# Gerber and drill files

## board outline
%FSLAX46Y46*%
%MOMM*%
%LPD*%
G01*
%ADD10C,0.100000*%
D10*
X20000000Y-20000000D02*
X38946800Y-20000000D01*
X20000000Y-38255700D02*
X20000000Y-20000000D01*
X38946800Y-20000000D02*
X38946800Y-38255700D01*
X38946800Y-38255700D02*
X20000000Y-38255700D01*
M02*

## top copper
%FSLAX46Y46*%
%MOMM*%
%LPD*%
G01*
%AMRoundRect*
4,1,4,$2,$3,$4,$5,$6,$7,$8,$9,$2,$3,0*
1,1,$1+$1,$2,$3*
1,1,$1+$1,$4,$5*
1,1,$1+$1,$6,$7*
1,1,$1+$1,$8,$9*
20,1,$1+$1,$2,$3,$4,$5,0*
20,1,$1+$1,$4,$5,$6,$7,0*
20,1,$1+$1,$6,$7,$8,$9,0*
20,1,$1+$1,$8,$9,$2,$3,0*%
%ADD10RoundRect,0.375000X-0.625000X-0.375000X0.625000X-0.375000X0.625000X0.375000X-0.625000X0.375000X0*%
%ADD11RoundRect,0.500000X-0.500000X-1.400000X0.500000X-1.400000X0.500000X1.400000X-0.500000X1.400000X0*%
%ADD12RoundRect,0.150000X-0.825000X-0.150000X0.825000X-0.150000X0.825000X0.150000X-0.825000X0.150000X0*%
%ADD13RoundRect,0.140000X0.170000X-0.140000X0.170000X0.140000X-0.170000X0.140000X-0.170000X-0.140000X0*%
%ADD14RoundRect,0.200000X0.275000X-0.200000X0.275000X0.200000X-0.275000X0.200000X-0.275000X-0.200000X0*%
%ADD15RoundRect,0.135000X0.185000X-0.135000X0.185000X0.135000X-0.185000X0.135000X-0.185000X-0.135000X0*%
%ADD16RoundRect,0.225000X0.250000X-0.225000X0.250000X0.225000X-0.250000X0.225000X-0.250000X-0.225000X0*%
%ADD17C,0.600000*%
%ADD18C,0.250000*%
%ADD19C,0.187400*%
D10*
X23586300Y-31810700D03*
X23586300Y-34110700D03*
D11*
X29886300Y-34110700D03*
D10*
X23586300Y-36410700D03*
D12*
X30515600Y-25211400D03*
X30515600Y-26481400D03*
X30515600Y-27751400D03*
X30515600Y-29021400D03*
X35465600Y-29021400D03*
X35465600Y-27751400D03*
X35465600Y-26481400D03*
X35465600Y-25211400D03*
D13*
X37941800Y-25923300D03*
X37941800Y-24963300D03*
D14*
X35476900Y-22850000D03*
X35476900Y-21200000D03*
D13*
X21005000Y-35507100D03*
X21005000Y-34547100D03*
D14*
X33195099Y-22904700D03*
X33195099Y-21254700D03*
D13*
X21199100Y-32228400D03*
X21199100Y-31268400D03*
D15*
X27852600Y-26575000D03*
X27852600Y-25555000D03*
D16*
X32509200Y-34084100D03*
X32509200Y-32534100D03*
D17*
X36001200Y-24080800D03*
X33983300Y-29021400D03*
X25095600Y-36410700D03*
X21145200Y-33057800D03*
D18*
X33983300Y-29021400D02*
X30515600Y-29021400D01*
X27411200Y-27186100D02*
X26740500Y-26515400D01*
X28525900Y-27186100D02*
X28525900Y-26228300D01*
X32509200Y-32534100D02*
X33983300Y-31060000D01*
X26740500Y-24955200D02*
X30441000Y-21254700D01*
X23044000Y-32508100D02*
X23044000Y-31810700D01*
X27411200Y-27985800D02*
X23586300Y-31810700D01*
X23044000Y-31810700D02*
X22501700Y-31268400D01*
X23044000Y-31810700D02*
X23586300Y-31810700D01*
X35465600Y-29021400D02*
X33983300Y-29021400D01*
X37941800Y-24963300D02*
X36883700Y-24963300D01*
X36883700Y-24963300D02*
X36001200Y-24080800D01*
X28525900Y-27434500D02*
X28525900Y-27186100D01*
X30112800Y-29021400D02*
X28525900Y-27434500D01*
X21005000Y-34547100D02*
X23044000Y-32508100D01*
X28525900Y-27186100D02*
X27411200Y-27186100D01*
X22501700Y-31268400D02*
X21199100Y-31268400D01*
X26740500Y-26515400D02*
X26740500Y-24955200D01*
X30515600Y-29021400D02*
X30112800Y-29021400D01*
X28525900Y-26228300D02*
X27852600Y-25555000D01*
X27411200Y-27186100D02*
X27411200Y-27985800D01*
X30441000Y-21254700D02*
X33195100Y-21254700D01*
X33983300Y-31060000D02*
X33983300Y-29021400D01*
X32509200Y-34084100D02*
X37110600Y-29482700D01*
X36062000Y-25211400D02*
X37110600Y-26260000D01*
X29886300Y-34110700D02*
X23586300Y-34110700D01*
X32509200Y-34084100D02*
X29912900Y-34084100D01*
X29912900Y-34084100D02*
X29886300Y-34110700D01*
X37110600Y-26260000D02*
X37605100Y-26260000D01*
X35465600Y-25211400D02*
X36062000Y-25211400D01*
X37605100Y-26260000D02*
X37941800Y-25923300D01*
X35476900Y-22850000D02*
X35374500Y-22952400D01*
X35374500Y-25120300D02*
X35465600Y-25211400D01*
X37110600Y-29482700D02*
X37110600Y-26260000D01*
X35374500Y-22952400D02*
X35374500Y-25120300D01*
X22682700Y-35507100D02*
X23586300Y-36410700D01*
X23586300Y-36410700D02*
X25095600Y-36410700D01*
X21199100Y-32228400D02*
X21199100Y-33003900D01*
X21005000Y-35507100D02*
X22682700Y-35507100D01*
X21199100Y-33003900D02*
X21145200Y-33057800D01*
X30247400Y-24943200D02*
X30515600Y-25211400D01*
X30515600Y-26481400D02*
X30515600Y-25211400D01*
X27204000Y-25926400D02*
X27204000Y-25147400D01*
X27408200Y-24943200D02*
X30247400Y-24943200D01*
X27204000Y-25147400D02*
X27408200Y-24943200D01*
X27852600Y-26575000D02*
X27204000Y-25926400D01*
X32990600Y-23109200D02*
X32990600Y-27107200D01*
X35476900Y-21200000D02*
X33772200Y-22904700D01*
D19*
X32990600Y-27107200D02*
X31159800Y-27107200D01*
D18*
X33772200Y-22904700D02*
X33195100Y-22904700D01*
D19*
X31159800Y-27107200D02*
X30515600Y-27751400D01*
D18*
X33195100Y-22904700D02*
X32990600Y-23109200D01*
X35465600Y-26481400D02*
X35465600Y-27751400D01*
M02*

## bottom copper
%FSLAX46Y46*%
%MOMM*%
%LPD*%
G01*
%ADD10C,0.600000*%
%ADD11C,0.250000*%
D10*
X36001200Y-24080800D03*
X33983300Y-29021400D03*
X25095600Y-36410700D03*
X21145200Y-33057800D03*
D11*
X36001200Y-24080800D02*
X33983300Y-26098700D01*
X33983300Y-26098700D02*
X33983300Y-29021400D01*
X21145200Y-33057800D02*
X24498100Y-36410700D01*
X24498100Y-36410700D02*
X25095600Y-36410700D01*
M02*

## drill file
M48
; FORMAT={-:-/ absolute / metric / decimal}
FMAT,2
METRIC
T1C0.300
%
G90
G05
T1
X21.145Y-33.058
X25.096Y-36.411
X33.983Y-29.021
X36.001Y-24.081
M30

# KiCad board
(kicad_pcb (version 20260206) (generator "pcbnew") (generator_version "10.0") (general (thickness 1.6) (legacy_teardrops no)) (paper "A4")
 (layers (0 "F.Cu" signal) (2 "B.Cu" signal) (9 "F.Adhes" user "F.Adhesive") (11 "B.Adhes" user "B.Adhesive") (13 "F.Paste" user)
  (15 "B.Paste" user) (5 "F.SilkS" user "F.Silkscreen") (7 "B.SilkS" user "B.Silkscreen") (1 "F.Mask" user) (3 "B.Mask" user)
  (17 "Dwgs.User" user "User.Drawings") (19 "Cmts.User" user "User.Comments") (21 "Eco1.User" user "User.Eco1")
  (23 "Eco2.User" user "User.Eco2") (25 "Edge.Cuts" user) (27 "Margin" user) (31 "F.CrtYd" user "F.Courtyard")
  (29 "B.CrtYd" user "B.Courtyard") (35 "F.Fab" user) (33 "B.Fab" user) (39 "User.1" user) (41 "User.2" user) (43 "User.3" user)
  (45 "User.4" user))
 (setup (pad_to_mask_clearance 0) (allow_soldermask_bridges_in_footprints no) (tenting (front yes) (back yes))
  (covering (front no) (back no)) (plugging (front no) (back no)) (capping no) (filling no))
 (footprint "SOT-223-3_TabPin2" (layer "F.Cu") (at 26.7363 34.1107)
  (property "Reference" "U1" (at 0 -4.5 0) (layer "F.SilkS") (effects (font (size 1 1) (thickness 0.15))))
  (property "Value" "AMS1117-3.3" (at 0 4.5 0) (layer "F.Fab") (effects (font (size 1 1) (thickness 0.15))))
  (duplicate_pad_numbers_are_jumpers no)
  (pad "1" smd roundrect (at -3.15 -2.3) (size 2 1.5) (layers "F.Cu" "F.Mask" "F.Paste") (roundrect_rratio 0.25) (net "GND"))
  (pad "2" smd roundrect (at -3.15 0) (size 2 1.5) (layers "F.Cu" "F.Mask" "F.Paste") (roundrect_rratio 0.25) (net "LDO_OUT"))
  (pad "2" smd roundrect (at 3.15 0) (size 2 3.8) (layers "F.Cu" "F.Mask" "F.Paste") (roundrect_rratio 0.25) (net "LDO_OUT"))
  (pad "3" smd roundrect (at -3.15 2.3) (size 2 1.5) (layers "F.Cu" "F.Mask" "F.Paste") (roundrect_rratio 0.25) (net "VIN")))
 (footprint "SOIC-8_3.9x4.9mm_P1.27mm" (layer "F.Cu") (at 32.9906 27.1164)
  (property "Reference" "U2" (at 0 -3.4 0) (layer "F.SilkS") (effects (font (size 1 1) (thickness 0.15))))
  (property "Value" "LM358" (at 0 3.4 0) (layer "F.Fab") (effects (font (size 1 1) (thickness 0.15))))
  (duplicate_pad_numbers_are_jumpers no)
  (pad "1" smd roundrect (at -2.475 -1.905) (size 1.95 0.6) (layers "F.Cu" "F.Mask" "F.Paste") (roundrect_rratio 0.25) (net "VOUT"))
  (pad "2" smd roundrect (at -2.475 -0.635) (size 1.95 0.6) (layers "F.Cu" "F.Mask" "F.Paste") (roundrect_rratio 0.25) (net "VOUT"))
  (pad "3" smd roundrect (at -2.475 0.635) (size 1.95 0.6) (layers "F.Cu" "F.Mask" "F.Paste") (roundrect_rratio 0.25) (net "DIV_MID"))
  (pad "4" smd roundrect (at -2.475 1.905) (size 1.95 0.6) (layers "F.Cu" "F.Mask" "F.Paste") (roundrect_rratio 0.25) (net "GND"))
  (pad "5" smd roundrect (at 2.475 1.905) (size 1.95 0.6) (layers "F.Cu" "F.Mask" "F.Paste") (roundrect_rratio 0.25) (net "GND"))
  (pad "6" smd roundrect (at 2.475 0.635) (size 1.95 0.6) (layers "F.Cu" "F.Mask" "F.Paste") (roundrect_rratio 0.25) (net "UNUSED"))
  (pad "7" smd roundrect (at 2.475 -0.635) (size 1.95 0.6) (layers "F.Cu" "F.Mask" "F.Paste") (roundrect_rratio 0.25) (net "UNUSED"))
  (pad "8" smd roundrect (at 2.475 -1.905) (size 1.95 0.6) (layers "F.Cu" "F.Mask" "F.Paste") (roundrect_rratio 0.25) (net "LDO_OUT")))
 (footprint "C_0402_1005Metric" (layer "F.Cu") (at 37.9418 25.4433 90)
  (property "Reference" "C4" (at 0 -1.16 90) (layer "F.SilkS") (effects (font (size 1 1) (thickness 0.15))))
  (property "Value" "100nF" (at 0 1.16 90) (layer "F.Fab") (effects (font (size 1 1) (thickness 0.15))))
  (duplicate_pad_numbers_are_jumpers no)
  (pad "1" smd roundrect (at -0.48 0 90) (size 0.56 0.62) (layers "F.Cu" "F.Mask" "F.Paste") (roundrect_rratio 0.25) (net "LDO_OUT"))
  (pad "2" smd roundrect (at 0.48 0 90) (size 0.56 0.62) (layers "F.Cu" "F.Mask" "F.Paste") (roundrect_rratio 0.25) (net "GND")))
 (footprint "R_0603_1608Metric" (layer "F.Cu") (at 35.4769 22.025 90)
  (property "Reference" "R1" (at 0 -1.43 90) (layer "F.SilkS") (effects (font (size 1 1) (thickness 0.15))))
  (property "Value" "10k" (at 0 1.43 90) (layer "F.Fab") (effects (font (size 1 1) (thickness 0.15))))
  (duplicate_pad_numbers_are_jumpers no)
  (pad "1" smd roundrect (at -0.825 0 90) (size 0.8 0.95) (layers "F.Cu" "F.Mask" "F.Paste") (roundrect_rratio 0.25) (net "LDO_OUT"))
  (pad "2" smd roundrect (at 0.825 0 90) (size 0.8 0.95) (layers "F.Cu" "F.Mask" "F.Paste") (roundrect_rratio 0.25) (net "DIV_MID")))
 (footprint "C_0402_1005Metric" (layer "F.Cu") (at 21.005 35.0271 90)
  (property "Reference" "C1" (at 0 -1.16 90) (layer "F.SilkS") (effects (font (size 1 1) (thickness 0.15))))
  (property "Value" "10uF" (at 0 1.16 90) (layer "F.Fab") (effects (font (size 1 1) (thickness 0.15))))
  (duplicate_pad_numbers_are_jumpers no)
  (pad "1" smd roundrect (at -0.48 0 90) (size 0.56 0.62) (layers "F.Cu" "F.Mask" "F.Paste") (roundrect_rratio 0.25) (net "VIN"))
  (pad "2" smd roundrect (at 0.48 0 90) (size 0.56 0.62) (layers "F.Cu" "F.Mask" "F.Paste") (roundrect_rratio 0.25) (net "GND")))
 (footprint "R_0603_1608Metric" (layer "F.Cu") (at 33.195099 22.0797 90)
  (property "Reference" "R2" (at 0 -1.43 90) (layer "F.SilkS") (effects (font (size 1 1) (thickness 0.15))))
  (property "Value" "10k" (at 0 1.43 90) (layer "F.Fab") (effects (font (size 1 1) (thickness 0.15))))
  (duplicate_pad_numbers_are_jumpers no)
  (pad "1" smd roundrect (at -0.825 0 90) (size 0.8 0.95) (layers "F.Cu" "F.Mask" "F.Paste") (roundrect_rratio 0.25) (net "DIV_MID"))
  (pad "2" smd roundrect (at 0.825 0 90) (size 0.8 0.95) (layers "F.Cu" "F.Mask" "F.Paste") (roundrect_rratio 0.25) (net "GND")))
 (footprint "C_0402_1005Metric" (layer "F.Cu") (at 21.1991 31.7484 90)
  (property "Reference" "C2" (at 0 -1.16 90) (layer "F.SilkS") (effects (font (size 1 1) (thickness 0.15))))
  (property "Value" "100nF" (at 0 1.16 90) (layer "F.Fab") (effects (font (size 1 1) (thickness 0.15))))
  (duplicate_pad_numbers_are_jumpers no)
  (pad "1" smd roundrect (at -0.48 0 90) (size 0.56 0.62) (layers "F.Cu" "F.Mask" "F.Paste") (roundrect_rratio 0.25) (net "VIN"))
  (pad "2" smd roundrect (at 0.48 0 90) (size 0.56 0.62) (layers "F.Cu" "F.Mask" "F.Paste") (roundrect_rratio 0.25) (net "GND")))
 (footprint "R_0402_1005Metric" (layer "F.Cu") (at 27.8526 26.065 90)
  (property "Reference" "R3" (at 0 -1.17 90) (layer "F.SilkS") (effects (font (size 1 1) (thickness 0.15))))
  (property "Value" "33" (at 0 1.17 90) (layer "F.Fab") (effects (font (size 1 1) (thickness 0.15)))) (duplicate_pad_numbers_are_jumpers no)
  (pad "1" smd roundrect (at -0.51 0 90) (size 0.54 0.64) (layers "F.Cu" "F.Mask" "F.Paste") (roundrect_rratio 0.25) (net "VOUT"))
  (pad "2" smd roundrect (at 0.51 0 90) (size 0.54 0.64) (layers "F.Cu" "F.Mask" "F.Paste") (roundrect_rratio 0.25) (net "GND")))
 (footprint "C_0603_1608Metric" (layer "F.Cu") (at 32.5092 33.3091 90)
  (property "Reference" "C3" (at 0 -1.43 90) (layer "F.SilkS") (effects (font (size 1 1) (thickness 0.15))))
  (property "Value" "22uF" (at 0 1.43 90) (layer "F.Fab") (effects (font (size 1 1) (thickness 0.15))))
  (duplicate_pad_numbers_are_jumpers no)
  (pad "1" smd roundrect (at -0.775 0 90) (size 0.9 0.95) (layers "F.Cu" "F.Mask" "F.Paste") (roundrect_rratio 0.25) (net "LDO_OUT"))
  (pad "2" smd roundrect (at 0.775 0 90) (size 0.9 0.95) (layers "F.Cu" "F.Mask" "F.Paste") (roundrect_rratio 0.25) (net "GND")))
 (gr_line (start 20 20) (end 38.9468 20) (stroke (width 0.1) (type default)) (layer "Edge.Cuts"))
 (gr_line (start 20 38.2557) (end 20 20) (stroke (width 0.1) (type default)) (layer "Edge.Cuts"))
 (gr_line (start 38.9468 20) (end 38.9468 38.2557) (stroke (width 0.1) (type default)) (layer "Edge.Cuts"))
 (gr_line (start 38.9468 38.2557) (end 20 38.2557) (stroke (width 0.1) (type default)) (layer "Edge.Cuts"))
 (segment (start 33.9833 29.0214) (end 30.5156 29.0214) (width 0.25) (layer "F.Cu") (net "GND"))
 (segment (start 27.4112 27.1861) (end 26.7405 26.5154) (width 0.25) (layer "F.Cu") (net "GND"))
 (segment (start 28.5259 27.1861) (end 28.5259 26.2283) (width 0.25) (layer "F.Cu") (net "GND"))
 (segment (start 32.5092 32.5341) (end 33.9833 31.06) (width 0.25) (layer "F.Cu") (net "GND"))
 (segment (start 26.7405 24.9552) (end 30.441 21.2547) (width 0.25) (layer "F.Cu") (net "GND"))
 (segment (start 23.044 32.5081) (end 23.044 31.8107) (width 0.25) (layer "F.Cu") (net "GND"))
 (segment (start 27.4112 27.9858) (end 23.5863 31.8107) (width 0.25) (layer "F.Cu") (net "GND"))
 (segment (start 23.044 31.8107) (end 22.5017 31.2684) (width 0.25) (layer "F.Cu") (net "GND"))
 (segment (start 23.044 31.8107) (end 23.5863 31.8107) (width 0.25) (layer "F.Cu") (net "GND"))
 (segment (start 35.4656 29.0214) (end 33.9833 29.0214) (width 0.25) (layer "F.Cu") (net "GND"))
 (segment (start 37.9418 24.9633) (end 36.8837 24.9633) (width 0.25) (layer "F.Cu") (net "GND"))
 (segment (start 36.8837 24.9633) (end 36.0012 24.0808) (width 0.25) (layer "F.Cu") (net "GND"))
 (segment (start 28.5259 27.4345) (end 28.5259 27.1861) (width 0.25) (layer "F.Cu") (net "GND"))
 (segment (start 30.1128 29.0214) (end 28.5259 27.4345) (width 0.25) (layer "F.Cu") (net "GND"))
 (segment (start 21.005 34.5471) (end 23.044 32.5081) (width 0.25) (layer "F.Cu") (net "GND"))
 (segment (start 28.5259 27.1861) (end 27.4112 27.1861) (width 0.25) (layer "F.Cu") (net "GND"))
 (segment (start 22.5017 31.2684) (end 21.1991 31.2684) (width 0.25) (layer "F.Cu") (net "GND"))
 (segment (start 26.7405 26.5154) (end 26.7405 24.9552) (width 0.25) (layer "F.Cu") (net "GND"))
 (segment (start 30.5156 29.0214) (end 30.1128 29.0214) (width 0.25) (layer "F.Cu") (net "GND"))
 (segment (start 28.5259 26.2283) (end 27.8526 25.555) (width 0.25) (layer "F.Cu") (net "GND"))
 (segment (start 27.4112 27.1861) (end 27.4112 27.9858) (width 0.25) (layer "F.Cu") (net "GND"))
 (segment (start 30.441 21.2547) (end 33.1951 21.2547) (width 0.25) (layer "F.Cu") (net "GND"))
 (segment (start 33.9833 31.06) (end 33.9833 29.0214) (width 0.25) (layer "F.Cu") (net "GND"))
 (via (at 36.0012 24.0808) (size 0.6) (drill 0.3) (layers "F.Cu" "B.Cu") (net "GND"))
 (via (at 33.9833 29.0214) (size 0.6) (drill 0.3) (layers "F.Cu" "B.Cu") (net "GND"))
 (segment (start 36.0012 24.0808) (end 33.9833 26.0987) (width 0.25) (layer "B.Cu") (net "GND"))
 (segment (start 33.9833 26.0987) (end 33.9833 29.0214) (width 0.25) (layer "B.Cu") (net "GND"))
 (segment (start 32.5092 34.0841) (end 37.1106 29.4827) (width 0.25) (layer "F.Cu") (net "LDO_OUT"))
 (segment (start 36.062 25.2114) (end 37.1106 26.26) (width 0.25) (layer "F.Cu") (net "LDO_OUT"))
 (segment (start 29.8863 34.1107) (end 23.5863 34.1107) (width 0.25) (layer "F.Cu") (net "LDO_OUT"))
 (segment (start 32.5092 34.0841) (end 29.9129 34.0841) (width 0.25) (layer "F.Cu") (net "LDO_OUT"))
 (segment (start 29.9129 34.0841) (end 29.8863 34.1107) (width 0.25) (layer "F.Cu") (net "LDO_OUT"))
 (segment (start 37.1106 26.26) (end 37.6051 26.26) (width 0.25) (layer "F.Cu") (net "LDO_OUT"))
 (segment (start 35.4656 25.2114) (end 36.062 25.2114) (width 0.25) (layer "F.Cu") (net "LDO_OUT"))
 (segment (start 37.6051 26.26) (end 37.9418 25.9233) (width 0.25) (layer "F.Cu") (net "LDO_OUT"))
 (segment (start 35.4769 22.85) (end 35.3745 22.9524) (width 0.25) (layer "F.Cu") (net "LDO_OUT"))
 (segment (start 35.3745 25.1203) (end 35.4656 25.2114) (width 0.25) (layer "F.Cu") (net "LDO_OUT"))
 (segment (start 37.1106 29.4827) (end 37.1106 26.26) (width 0.25) (layer "F.Cu") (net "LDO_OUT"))
 (segment (start 35.3745 22.9524) (end 35.3745 25.1203) (width 0.25) (layer "F.Cu") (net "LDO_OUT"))
 (segment (start 22.6827 35.5071) (end 23.5863 36.4107) (width 0.25) (layer "F.Cu") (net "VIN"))
 (segment (start 23.5863 36.4107) (end 25.0956 36.4107) (width 0.25) (layer "F.Cu") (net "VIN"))
 (segment (start 21.1991 32.2284) (end 21.1991 33.0039) (width 0.25) (layer "F.Cu") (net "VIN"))
 (segment (start 21.005 35.5071) (end 22.6827 35.5071) (width 0.25) (layer "F.Cu") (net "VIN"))
 (segment (start 21.1991 33.0039) (end 21.1452 33.0578) (width 0.25) (layer "F.Cu") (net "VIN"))
 (via (at 25.0956 36.4107) (size 0.6) (drill 0.3) (layers "F.Cu" "B.Cu") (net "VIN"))
 (via (at 21.1452 33.0578) (size 0.6) (drill 0.3) (layers "F.Cu" "B.Cu") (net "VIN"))
 (segment (start 21.1452 33.0578) (end 24.4981 36.4107) (width 0.25) (layer "B.Cu") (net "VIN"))
 (segment (start 24.4981 36.4107) (end 25.0956 36.4107) (width 0.25) (layer "B.Cu") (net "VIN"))
 (segment (start 30.2474 24.9432) (end 30.5156 25.2114) (width 0.25) (layer "F.Cu") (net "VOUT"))
 (segment (start 30.5156 26.4814) (end 30.5156 25.2114) (width 0.25) (layer "F.Cu") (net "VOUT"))
 (segment (start 27.204 25.9264) (end 27.204 25.1474) (width 0.25) (layer "F.Cu") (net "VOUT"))
 (segment (start 27.4082 24.9432) (end 30.2474 24.9432) (width 0.25) (layer "F.Cu") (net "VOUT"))
 (segment (start 27.204 25.1474) (end 27.4082 24.9432) (width 0.25) (layer "F.Cu") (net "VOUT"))
 (segment (start 27.8526 26.575) (end 27.204 25.9264) (width 0.25) (layer "F.Cu") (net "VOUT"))
 (segment (start 32.9906 23.1092) (end 32.9906 27.1072) (width 0.25) (layer "F.Cu") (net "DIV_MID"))
 (segment (start 35.4769 21.2) (end 33.7722 22.9047) (width 0.25) (layer "F.Cu") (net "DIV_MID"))
 (segment (start 32.9906 27.1072) (end 31.1598 27.1072) (width 0.1874) (layer "F.Cu") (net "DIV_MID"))
 (segment (start 33.7722 22.9047) (end 33.1951 22.9047) (width 0.25) (layer "F.Cu") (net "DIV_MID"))
 (segment (start 31.1598 27.1072) (end 30.5156 27.7514) (width 0.1874) (layer "F.Cu") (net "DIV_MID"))
 (segment (start 33.1951 22.9047) (end 32.9906 23.1092) (width 0.25) (layer "F.Cu") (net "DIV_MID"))
 (segment (start 35.4656 26.4814) (end 35.4656 27.7514) (width 0.25) (layer "F.Cu") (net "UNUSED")))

